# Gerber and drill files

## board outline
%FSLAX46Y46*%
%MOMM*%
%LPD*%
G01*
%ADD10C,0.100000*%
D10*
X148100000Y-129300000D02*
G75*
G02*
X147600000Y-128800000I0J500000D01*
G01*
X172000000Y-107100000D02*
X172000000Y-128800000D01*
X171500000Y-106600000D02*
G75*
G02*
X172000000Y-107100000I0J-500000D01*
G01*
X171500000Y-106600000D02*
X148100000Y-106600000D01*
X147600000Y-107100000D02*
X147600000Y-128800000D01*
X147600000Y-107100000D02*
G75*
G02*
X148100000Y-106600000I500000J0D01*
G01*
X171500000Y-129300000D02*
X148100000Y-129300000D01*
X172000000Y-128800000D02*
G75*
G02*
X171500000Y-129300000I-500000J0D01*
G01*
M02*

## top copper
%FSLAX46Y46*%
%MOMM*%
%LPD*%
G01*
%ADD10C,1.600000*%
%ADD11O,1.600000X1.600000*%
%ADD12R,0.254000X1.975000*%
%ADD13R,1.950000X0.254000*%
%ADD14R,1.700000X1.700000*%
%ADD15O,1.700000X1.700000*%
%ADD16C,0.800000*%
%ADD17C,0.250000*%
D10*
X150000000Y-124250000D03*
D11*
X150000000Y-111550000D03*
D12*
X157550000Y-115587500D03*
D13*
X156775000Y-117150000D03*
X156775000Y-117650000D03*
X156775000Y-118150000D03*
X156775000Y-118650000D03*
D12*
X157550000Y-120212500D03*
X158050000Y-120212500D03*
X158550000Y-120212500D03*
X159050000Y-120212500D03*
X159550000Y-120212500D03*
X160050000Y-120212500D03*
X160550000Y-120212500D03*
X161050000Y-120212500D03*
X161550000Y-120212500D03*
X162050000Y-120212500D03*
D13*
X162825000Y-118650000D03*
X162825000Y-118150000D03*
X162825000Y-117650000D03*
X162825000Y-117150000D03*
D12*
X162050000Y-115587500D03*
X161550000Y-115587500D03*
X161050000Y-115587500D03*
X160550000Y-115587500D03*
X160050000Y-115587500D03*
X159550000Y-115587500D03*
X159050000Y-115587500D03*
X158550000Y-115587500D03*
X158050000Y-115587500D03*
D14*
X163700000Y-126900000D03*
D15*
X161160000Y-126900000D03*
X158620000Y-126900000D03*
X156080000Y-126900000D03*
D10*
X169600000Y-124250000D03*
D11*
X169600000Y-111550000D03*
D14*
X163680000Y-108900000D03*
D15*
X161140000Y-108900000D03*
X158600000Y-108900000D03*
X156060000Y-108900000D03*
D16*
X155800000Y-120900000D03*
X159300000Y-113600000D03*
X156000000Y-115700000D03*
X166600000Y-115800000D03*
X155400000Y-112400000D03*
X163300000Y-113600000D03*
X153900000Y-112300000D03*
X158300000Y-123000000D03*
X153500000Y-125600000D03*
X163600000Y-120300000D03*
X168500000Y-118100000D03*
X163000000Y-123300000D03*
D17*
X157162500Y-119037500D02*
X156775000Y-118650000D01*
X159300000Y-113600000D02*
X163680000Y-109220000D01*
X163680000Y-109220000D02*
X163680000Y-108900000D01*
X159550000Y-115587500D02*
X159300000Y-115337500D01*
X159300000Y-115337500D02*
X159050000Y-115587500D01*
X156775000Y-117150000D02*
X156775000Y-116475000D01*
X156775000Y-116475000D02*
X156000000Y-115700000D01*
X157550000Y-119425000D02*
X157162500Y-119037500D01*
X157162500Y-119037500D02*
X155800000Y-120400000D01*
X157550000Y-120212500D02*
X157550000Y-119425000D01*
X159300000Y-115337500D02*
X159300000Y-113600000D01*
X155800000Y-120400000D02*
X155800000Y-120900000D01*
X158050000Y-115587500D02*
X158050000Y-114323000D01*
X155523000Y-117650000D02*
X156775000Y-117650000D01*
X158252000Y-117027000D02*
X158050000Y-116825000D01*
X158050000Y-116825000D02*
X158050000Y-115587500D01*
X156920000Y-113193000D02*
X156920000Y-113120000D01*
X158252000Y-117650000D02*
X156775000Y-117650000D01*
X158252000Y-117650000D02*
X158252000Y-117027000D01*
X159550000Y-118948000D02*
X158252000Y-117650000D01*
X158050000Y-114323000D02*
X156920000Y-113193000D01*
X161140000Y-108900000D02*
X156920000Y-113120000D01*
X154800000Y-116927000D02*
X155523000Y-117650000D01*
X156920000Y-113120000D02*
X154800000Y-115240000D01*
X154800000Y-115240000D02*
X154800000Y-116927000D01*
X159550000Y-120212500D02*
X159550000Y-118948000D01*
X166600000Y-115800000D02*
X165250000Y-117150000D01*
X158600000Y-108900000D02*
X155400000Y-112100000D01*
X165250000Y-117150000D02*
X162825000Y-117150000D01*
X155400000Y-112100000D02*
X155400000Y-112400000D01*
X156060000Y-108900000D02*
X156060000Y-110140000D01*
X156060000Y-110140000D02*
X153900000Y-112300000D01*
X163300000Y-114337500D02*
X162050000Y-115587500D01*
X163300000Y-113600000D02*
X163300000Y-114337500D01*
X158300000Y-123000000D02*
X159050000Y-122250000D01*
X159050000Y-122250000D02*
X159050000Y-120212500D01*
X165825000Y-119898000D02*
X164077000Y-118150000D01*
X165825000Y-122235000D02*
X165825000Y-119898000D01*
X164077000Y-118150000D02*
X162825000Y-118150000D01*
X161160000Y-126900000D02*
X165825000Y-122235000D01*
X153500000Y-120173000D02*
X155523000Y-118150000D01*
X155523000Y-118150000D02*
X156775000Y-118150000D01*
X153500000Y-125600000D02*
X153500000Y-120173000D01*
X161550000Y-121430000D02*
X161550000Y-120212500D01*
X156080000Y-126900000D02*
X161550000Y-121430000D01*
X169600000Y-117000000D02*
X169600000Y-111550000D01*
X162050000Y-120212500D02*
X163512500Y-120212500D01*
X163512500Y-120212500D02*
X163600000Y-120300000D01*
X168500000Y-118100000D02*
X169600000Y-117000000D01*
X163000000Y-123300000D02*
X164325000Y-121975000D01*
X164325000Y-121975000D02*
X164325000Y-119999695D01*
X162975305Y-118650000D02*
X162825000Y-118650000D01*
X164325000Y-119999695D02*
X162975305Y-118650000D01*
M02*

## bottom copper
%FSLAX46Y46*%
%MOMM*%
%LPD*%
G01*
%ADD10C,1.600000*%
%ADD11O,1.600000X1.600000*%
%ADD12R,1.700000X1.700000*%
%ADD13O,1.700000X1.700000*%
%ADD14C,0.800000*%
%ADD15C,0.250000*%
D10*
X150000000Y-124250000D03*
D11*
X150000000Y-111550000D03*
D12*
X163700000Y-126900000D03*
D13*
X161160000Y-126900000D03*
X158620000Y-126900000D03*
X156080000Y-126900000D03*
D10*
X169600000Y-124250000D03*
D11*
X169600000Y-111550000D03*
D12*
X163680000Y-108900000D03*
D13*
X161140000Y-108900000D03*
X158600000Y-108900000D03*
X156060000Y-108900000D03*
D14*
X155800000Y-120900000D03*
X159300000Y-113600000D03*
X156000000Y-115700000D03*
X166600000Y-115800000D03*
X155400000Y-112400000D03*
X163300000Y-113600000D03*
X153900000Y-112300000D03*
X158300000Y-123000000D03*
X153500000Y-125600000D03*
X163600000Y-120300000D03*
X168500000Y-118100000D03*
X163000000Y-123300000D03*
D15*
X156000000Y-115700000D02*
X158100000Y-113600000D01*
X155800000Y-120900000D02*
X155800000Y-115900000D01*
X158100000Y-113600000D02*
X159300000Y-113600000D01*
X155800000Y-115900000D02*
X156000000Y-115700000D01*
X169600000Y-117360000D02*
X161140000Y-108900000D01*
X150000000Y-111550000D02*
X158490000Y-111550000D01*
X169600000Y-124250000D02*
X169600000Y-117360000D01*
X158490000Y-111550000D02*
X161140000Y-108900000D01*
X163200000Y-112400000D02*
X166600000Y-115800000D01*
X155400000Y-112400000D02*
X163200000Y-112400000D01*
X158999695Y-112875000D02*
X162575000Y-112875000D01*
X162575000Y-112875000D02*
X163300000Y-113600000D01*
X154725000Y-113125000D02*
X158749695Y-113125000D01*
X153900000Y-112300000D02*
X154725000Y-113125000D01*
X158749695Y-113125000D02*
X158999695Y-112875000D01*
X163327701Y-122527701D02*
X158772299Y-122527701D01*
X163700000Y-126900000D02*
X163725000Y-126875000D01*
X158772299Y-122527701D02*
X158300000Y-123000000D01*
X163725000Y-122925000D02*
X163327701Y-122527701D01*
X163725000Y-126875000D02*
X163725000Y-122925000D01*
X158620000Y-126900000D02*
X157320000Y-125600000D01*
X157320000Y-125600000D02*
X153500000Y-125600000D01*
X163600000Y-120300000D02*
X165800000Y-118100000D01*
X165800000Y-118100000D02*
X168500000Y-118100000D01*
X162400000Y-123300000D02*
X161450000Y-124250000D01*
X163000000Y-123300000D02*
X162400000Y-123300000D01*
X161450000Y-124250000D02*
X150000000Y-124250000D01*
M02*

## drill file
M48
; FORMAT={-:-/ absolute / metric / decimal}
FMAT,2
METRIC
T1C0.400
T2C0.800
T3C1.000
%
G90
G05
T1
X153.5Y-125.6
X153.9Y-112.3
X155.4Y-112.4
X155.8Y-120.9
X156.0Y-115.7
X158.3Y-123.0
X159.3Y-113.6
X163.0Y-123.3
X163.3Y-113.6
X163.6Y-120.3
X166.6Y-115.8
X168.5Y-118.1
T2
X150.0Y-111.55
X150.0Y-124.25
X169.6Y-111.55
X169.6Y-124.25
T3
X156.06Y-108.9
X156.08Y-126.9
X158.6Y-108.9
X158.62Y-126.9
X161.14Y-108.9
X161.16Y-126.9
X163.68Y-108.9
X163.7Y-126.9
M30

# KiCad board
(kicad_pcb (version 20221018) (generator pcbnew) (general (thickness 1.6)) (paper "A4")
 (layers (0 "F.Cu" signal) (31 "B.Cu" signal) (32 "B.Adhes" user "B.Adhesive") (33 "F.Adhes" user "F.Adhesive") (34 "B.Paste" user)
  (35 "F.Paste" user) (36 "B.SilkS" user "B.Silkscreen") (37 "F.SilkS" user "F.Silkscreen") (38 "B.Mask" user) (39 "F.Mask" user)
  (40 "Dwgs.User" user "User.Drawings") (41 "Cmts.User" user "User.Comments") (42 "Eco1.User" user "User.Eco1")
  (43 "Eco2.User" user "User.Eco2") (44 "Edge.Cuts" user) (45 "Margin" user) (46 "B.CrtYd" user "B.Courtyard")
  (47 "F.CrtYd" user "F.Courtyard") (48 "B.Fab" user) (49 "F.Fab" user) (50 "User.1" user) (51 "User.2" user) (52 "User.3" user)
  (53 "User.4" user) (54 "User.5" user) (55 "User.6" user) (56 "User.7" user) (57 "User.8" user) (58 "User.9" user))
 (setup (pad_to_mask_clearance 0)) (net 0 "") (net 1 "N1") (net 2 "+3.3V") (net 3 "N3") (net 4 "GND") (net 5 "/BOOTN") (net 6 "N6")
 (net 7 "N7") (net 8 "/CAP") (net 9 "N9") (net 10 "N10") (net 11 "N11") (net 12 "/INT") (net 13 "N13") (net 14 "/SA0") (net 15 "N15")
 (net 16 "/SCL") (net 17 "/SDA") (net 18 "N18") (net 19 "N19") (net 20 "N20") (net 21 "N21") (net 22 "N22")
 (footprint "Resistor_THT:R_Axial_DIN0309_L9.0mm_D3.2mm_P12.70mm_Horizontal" (layer "F.Cu") (at 150 124.25 90)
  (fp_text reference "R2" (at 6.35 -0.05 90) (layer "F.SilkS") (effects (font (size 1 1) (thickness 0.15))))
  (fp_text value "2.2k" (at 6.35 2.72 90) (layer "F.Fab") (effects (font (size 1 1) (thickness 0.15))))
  (pad "1" thru_hole circle (at 0 0 90) (size 1.6 1.6) (drill 0.8) (layers "*.Cu" "*.Mask") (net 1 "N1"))
  (pad "2" thru_hole oval (at 12.7 0 90) (size 1.6 1.6) (drill 0.8) (layers "*.Cu" "*.Mask") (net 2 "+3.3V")))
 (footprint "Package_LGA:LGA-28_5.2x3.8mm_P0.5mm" (layer "F.Cu") (at 159.8 117.9)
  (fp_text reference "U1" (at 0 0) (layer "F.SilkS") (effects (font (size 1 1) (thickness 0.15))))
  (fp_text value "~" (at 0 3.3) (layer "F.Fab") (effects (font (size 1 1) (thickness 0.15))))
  (pad "1" smd rect (at -2.25 -2.3125) (size 0.254 1.975) (layers "F.Cu" "F.Paste" "F.Mask") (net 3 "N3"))
  (pad "2" smd rect (at -3.025 -0.75 90) (size 0.254 1.95) (layers "F.Cu" "F.Paste" "F.Mask") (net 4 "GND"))
  (pad "3" smd rect (at -3.025 -0.25 90) (size 0.254 1.95) (layers "F.Cu" "F.Paste" "F.Mask") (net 2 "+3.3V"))
  (pad "4" smd rect (at -3.025 0.25 90) (size 0.254 1.95) (layers "F.Cu" "F.Paste" "F.Mask") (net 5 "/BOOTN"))
  (pad "5" smd rect (at -3.025 0.75 90) (size 0.254 1.95) (layers "F.Cu" "F.Paste" "F.Mask") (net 4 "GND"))
  (pad "6" smd rect (at -2.25 2.3125) (size 0.254 1.975) (layers "F.Cu" "F.Paste" "F.Mask") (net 4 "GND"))
  (pad "7" smd rect (at -1.75 2.3125) (size 0.254 1.975) (layers "F.Cu" "F.Paste" "F.Mask") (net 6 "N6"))
  (pad "8" smd rect (at -1.25 2.3125) (size 0.254 1.975) (layers "F.Cu" "F.Paste" "F.Mask") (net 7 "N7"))
  (pad "9" smd rect (at -0.75 2.3125) (size 0.254 1.975) (layers "F.Cu" "F.Paste" "F.Mask") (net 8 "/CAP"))
  (pad "10" smd rect (at -0.25 2.3125) (size 0.254 1.975) (layers "F.Cu" "F.Paste" "F.Mask") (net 2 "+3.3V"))
  (pad "11" smd rect (at 0.25 2.3125) (size 0.254 1.975) (layers "F.Cu" "F.Paste" "F.Mask") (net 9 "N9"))
  (pad "12" smd rect (at 0.75 2.3125) (size 0.254 1.975) (layers "F.Cu" "F.Paste" "F.Mask") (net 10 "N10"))
  (pad "13" smd rect (at 1.25 2.3125) (size 0.254 1.975) (layers "F.Cu" "F.Paste" "F.Mask") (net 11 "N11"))
  (pad "14" smd rect (at 1.75 2.3125) (size 0.254 1.975) (layers "F.Cu" "F.Paste" "F.Mask") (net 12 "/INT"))
  (pad "15" smd rect (at 2.25 2.3125) (size 0.254 1.975) (layers "F.Cu" "F.Paste" "F.Mask") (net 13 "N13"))
  (pad "16" smd rect (at 3.025 0.75 90) (size 0.254 1.95) (layers "F.Cu" "F.Paste" "F.Mask") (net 1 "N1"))
  (pad "17" smd rect (at 3.025 0.25 90) (size 0.254 1.95) (layers "F.Cu" "F.Paste" "F.Mask") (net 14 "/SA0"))
  (pad "18" smd rect (at 3.025 -0.25 90) (size 0.254 1.95) (layers "F.Cu" "F.Paste" "F.Mask") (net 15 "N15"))
  (pad "19" smd rect (at 3.025 -0.75 90) (size 0.254 1.95) (layers "F.Cu" "F.Paste" "F.Mask") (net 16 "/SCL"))
  (pad "20" smd rect (at 2.25 -2.3125) (size 0.254 1.975) (layers "F.Cu" "F.Paste" "F.Mask") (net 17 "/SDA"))
  (pad "21" smd rect (at 1.75 -2.3125) (size 0.254 1.975) (layers "F.Cu" "F.Paste" "F.Mask") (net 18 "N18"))
  (pad "22" smd rect (at 1.25 -2.3125) (size 0.254 1.975) (layers "F.Cu" "F.Paste" "F.Mask") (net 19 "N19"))
  (pad "23" smd rect (at 0.75 -2.3125) (size 0.254 1.975) (layers "F.Cu" "F.Paste" "F.Mask") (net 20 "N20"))
  (pad "24" smd rect (at 0.25 -2.3125) (size 0.254 1.975) (layers "F.Cu" "F.Paste" "F.Mask") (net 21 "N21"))
  (pad "25" smd rect (at -0.25 -2.3125) (size 0.254 1.975) (layers "F.Cu" "F.Paste" "F.Mask") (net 4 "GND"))
  (pad "26" smd rect (at -0.75 -2.3125) (size 0.254 1.975) (layers "F.Cu" "F.Paste" "F.Mask") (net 4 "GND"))
  (pad "27" smd rect (at -1.25 -2.3125) (size 0.254 1.975) (layers "F.Cu" "F.Paste" "F.Mask") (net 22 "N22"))
  (pad "28" smd rect (at -1.75 -2.3125) (size 0.254 1.975) (layers "F.Cu" "F.Paste" "F.Mask") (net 2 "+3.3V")))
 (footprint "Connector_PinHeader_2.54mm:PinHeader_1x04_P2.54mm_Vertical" (layer "F.Cu") (at 163.7 126.9 -90)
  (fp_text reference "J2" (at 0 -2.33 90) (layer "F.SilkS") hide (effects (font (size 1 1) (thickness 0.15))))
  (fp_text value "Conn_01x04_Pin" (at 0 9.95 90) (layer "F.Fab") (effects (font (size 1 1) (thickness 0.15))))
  (pad "1" thru_hole rect (at 0 0 270) (size 1.7 1.7) (drill 1) (layers "*.Cu" "*.Mask") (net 8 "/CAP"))
  (pad "2" thru_hole oval (at 0 2.54 270) (size 1.7 1.7) (drill 1) (layers "*.Cu" "*.Mask") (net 14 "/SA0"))
  (pad "3" thru_hole oval (at 0 5.08 270) (size 1.7 1.7) (drill 1) (layers "*.Cu" "*.Mask") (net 5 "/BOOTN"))
  (pad "4" thru_hole oval (at 0 7.62 270) (size 1.7 1.7) (drill 1) (layers "*.Cu" "*.Mask") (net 12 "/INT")))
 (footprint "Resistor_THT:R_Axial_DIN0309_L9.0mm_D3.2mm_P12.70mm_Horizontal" (layer "F.Cu") (at 169.6 124.25 90)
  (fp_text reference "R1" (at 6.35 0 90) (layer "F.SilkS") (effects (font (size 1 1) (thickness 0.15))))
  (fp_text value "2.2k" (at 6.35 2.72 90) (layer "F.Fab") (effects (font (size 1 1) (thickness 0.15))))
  (pad "1" thru_hole circle (at 0 0 90) (size 1.6 1.6) (drill 0.8) (layers "*.Cu" "*.Mask") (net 2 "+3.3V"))
  (pad "2" thru_hole oval (at 12.7 0 90) (size 1.6 1.6) (drill 0.8) (layers "*.Cu" "*.Mask") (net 13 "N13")))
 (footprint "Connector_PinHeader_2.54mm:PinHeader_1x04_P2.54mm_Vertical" (layer "F.Cu") (at 163.68 108.9 -90)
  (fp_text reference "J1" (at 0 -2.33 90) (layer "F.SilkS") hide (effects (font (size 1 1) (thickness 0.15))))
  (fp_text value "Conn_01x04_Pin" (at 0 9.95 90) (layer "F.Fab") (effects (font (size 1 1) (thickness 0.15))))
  (pad "1" thru_hole rect (at 0 0 270) (size 1.7 1.7) (drill 1) (layers "*.Cu" "*.Mask") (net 4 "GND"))
  (pad "2" thru_hole oval (at 0 2.54 270) (size 1.7 1.7) (drill 1) (layers "*.Cu" "*.Mask") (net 2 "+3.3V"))
  (pad "3" thru_hole oval (at 0 5.08 270) (size 1.7 1.7) (drill 1) (layers "*.Cu" "*.Mask") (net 16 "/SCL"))
  (pad "4" thru_hole oval (at 0 7.62 270) (size 1.7 1.7) (drill 1) (layers "*.Cu" "*.Mask") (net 17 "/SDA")))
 (gr_arc (start 148.1 129.3) (mid 147.746447 129.153553) (end 147.6 128.8) (stroke (width 0.1) (type default)) (layer "Edge.Cuts"))
 (gr_line (start 172 107.1) (end 172 128.8) (stroke (width 0.1) (type default)) (layer "Edge.Cuts"))
 (gr_arc (start 171.5 106.6) (mid 171.853553 106.746447) (end 172 107.1) (stroke (width 0.1) (type default)) (layer "Edge.Cuts"))
 (gr_line (start 171.5 106.6) (end 148.1 106.6) (stroke (width 0.1) (type default)) (layer "Edge.Cuts"))
 (gr_line (start 147.6 107.1) (end 147.6 128.8) (stroke (width 0.1) (type default)) (layer "Edge.Cuts"))
 (gr_arc (start 147.6 107.1) (mid 147.746447 106.746447) (end 148.1 106.6) (stroke (width 0.1) (type default)) (layer "Edge.Cuts"))
 (gr_line (start 171.5 129.3) (end 148.1 129.3) (stroke (width 0.1) (type default)) (layer "Edge.Cuts"))
 (gr_arc (start 172 128.8) (mid 171.853553 129.153553) (end 171.5 129.3) (stroke (width 0.1) (type default)) (layer "Edge.Cuts"))
 (segment (start 157.1625 119.0375) (end 156.775 118.65) (width 0.25) (layer "F.Cu") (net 4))
 (segment (start 159.3 113.6) (end 163.68 109.22) (width 0.25) (layer "F.Cu") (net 4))
 (segment (start 163.68 109.22) (end 163.68 108.9) (width 0.25) (layer "F.Cu") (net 4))
 (segment (start 159.55 115.5875) (end 159.3 115.3375) (width 0.25) (layer "F.Cu") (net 4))
 (segment (start 159.3 115.3375) (end 159.05 115.5875) (width 0.25) (layer "F.Cu") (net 4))
 (segment (start 156.775 117.15) (end 156.775 116.475) (width 0.25) (layer "F.Cu") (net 4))
 (segment (start 156.775 116.475) (end 156 115.7) (width 0.25) (layer "F.Cu") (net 4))
 (segment (start 157.55 119.425) (end 157.1625 119.0375) (width 0.25) (layer "F.Cu") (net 4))
 (segment (start 157.1625 119.0375) (end 155.8 120.4) (width 0.25) (layer "F.Cu") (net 4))
 (segment (start 157.55 120.2125) (end 157.55 119.425) (width 0.25) (layer "F.Cu") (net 4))
 (segment (start 159.3 115.3375) (end 159.3 113.6) (width 0.25) (layer "F.Cu") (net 4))
 (segment (start 155.8 120.4) (end 155.8 120.9) (width 0.25) (layer "F.Cu") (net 4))
 (via (at 155.8 120.9) (size 0.8) (drill 0.4) (layers "F.Cu" "B.Cu") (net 4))
 (via (at 159.3 113.6) (size 0.8) (drill 0.4) (layers "F.Cu" "B.Cu") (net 4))
 (via (at 156 115.7) (size 0.8) (drill 0.4) (layers "F.Cu" "B.Cu") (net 4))
 (segment (start 156 115.7) (end 158.1 113.6) (width 0.25) (layer "B.Cu") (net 4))
 (segment (start 155.8 120.9) (end 155.8 115.9) (width 0.25) (layer "B.Cu") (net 4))
 (segment (start 158.1 113.6) (end 159.3 113.6) (width 0.25) (layer "B.Cu") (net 4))
 (segment (start 155.8 115.9) (end 156 115.7) (width 0.25) (layer "B.Cu") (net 4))
 (segment (start 158.05 115.5875) (end 158.05 114.323) (width 0.25) (layer "F.Cu") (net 2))
 (segment (start 155.523 117.65) (end 156.775 117.65) (width 0.25) (layer "F.Cu") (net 2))
 (segment (start 158.252 117.027) (end 158.05 116.825) (width 0.25) (layer "F.Cu") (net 2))
 (segment (start 158.05 116.825) (end 158.05 115.5875) (width 0.25) (layer "F.Cu") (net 2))
 (segment (start 156.92 113.193) (end 156.92 113.12) (width 0.25) (layer "F.Cu") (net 2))
 (segment (start 158.252 117.65) (end 156.775 117.65) (width 0.25) (layer "F.Cu") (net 2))
 (segment (start 158.252 117.65) (end 158.252 117.027) (width 0.25) (layer "F.Cu") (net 2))
 (segment (start 159.55 118.948) (end 158.252 117.65) (width 0.25) (layer "F.Cu") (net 2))
 (segment (start 158.05 114.323) (end 156.92 113.193) (width 0.25) (layer "F.Cu") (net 2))
 (segment (start 161.14 108.9) (end 156.92 113.12) (width 0.25) (layer "F.Cu") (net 2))
 (segment (start 154.8 116.927) (end 155.523 117.65) (width 0.25) (layer "F.Cu") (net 2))
 (segment (start 156.92 113.12) (end 154.8 115.24) (width 0.25) (layer "F.Cu") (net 2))
 (segment (start 154.8 115.24) (end 154.8 116.927) (width 0.25) (layer "F.Cu") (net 2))
 (segment (start 159.55 120.2125) (end 159.55 118.948) (width 0.25) (layer "F.Cu") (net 2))
 (segment (start 169.6 117.36) (end 161.14 108.9) (width 0.25) (layer "B.Cu") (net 2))
 (segment (start 150 111.55) (end 158.49 111.55) (width 0.25) (layer "B.Cu") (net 2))
 (segment (start 169.6 124.25) (end 169.6 117.36) (width 0.25) (layer "B.Cu") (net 2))
 (segment (start 158.49 111.55) (end 161.14 108.9) (width 0.25) (layer "B.Cu") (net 2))
 (segment (start 166.6 115.8) (end 165.25 117.15) (width 0.25) (layer "F.Cu") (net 16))
 (segment (start 158.6 108.9) (end 155.4 112.1) (width 0.25) (layer "F.Cu") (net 16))
 (segment (start 165.25 117.15) (end 162.825 117.15) (width 0.25) (layer "F.Cu") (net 16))
 (segment (start 155.4 112.1) (end 155.4 112.4) (width 0.25) (layer "F.Cu") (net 16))
 (via (at 166.6 115.8) (size 0.8) (drill 0.4) (layers "F.Cu" "B.Cu") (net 16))
 (via (at 155.4 112.4) (size 0.8) (drill 0.4) (layers "F.Cu" "B.Cu") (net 16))
 (segment (start 163.2 112.4) (end 166.6 115.8) (width 0.25) (layer "B.Cu") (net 16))
 (segment (start 155.4 112.4) (end 163.2 112.4) (width 0.25) (layer "B.Cu") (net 16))
 (segment (start 156.06 108.9) (end 156.06 110.14) (width 0.25) (layer "F.Cu") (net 17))
 (segment (start 156.06 110.14) (end 153.9 112.3) (width 0.25) (layer "F.Cu") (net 17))
 (segment (start 163.3 114.3375) (end 162.05 115.5875) (width 0.25) (layer "F.Cu") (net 17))
 (segment (start 163.3 113.6) (end 163.3 114.3375) (width 0.25) (layer "F.Cu") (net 17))
 (via (at 163.3 113.6) (size 0.8) (drill 0.4) (layers "F.Cu" "B.Cu") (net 17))
 (via (at 153.9 112.3) (size 0.8) (drill 0.4) (layers "F.Cu" "B.Cu") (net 17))
 (segment (start 158.999695 112.875) (end 162.575 112.875) (width 0.25) (layer "B.Cu") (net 17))
 (segment (start 162.575 112.875) (end 163.3 113.6) (width 0.25) (layer "B.Cu") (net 17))
 (segment (start 154.725 113.125) (end 158.749695 113.125) (width 0.25) (layer "B.Cu") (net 17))
 (segment (start 153.9 112.3) (end 154.725 113.125) (width 0.25) (layer "B.Cu") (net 17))
 (segment (start 158.749695 113.125) (end 158.999695 112.875) (width 0.25) (layer "B.Cu") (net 17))
 (segment (start 158.3 123) (end 159.05 122.25) (width 0.25) (layer "F.Cu") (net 8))
 (segment (start 159.05 122.25) (end 159.05 120.2125) (width 0.25) (layer "F.Cu") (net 8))
 (via (at 158.3 123) (size 0.8) (drill 0.4) (layers "F.Cu" "B.Cu") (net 8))
 (segment (start 163.327701 122.527701) (end 158.772299 122.527701) (width 0.25) (layer "B.Cu") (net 8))
 (segment (start 163.7 126.9) (end 163.725 126.875) (width 0.25) (layer "B.Cu") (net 8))
 (segment (start 158.772299 122.527701) (end 158.3 123) (width 0.25) (layer "B.Cu") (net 8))
 (segment (start 163.725 122.925) (end 163.327701 122.527701) (width 0.25) (layer "B.Cu") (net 8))
 (segment (start 163.725 126.875) (end 163.725 122.925) (width 0.25) (layer "B.Cu") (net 8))
 (segment (start 165.825 119.898) (end 164.077 118.15) (width 0.25) (layer "F.Cu") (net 14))
 (segment (start 165.825 122.235) (end 165.825 119.898) (width 0.25) (layer "F.Cu") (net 14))
 (segment (start 164.077 118.15) (end 162.825 118.15) (width 0.25) (layer "F.Cu") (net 14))
 (segment (start 161.16 126.9) (end 165.825 122.235) (width 0.25) (layer "F.Cu") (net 14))
 (segment (start 153.5 120.173) (end 155.523 118.15) (width 0.25) (layer "F.Cu") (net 5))
 (segment (start 155.523 118.15) (end 156.775 118.15) (width 0.25) (layer "F.Cu") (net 5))
 (segment (start 153.5 125.6) (end 153.5 120.173) (width 0.25) (layer "F.Cu") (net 5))
 (via (at 153.5 125.6) (size 0.8) (drill 0.4) (layers "F.Cu" "B.Cu") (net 5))
 (segment (start 158.62 126.9) (end 157.32 125.6) (width 0.25) (layer "B.Cu") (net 5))
 (segment (start 157.32 125.6) (end 153.5 125.6) (width 0.25) (layer "B.Cu") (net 5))
 (segment (start 161.55 121.43) (end 161.55 120.2125) (width 0.25) (layer "F.Cu") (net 12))
 (segment (start 156.08 126.9) (end 161.55 121.43) (width 0.25) (layer "F.Cu") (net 12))
 (segment (start 169.6 117) (end 169.6 111.55) (width 0.25) (layer "F.Cu") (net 13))
 (segment (start 162.05 120.2125) (end 163.5125 120.2125) (width 0.25) (layer "F.Cu") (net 13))
 (segment (start 163.5125 120.2125) (end 163.6 120.3) (width 0.25) (layer "F.Cu") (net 13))
 (segment (start 168.5 118.1) (end 169.6 117) (width 0.25) (layer "F.Cu") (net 13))
 (via (at 163.6 120.3) (size 0.8) (drill 0.4) (layers "F.Cu" "B.Cu") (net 13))
 (via (at 168.5 118.1) (size 0.8) (drill 0.4) (layers "F.Cu" "B.Cu") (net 13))
 (segment (start 163.6 120.3) (end 165.8 118.1) (width 0.25) (layer "B.Cu") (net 13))
 (segment (start 165.8 118.1) (end 168.5 118.1) (width 0.25) (layer "B.Cu") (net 13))
 (segment (start 163 123.3) (end 164.325 121.975) (width 0.25) (layer "F.Cu") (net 1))
 (segment (start 164.325 121.975) (end 164.325 119.999695) (width 0.25) (layer "F.Cu") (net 1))
 (segment (start 162.975305 118.65) (end 162.825 118.65) (width 0.25) (layer "F.Cu") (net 1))
 (segment (start 164.325 119.999695) (end 162.975305 118.65) (width 0.25) (layer "F.Cu") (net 1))
 (via (at 163 123.3) (size 0.8) (drill 0.4) (layers "F.Cu" "B.Cu") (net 1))
 (segment (start 162.4 123.3) (end 161.45 124.25) (width 0.25) (layer "B.Cu") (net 1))
 (segment (start 163 123.3) (end 162.4 123.3) (width 0.25) (layer "B.Cu") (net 1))
 (segment (start 161.45 124.25) (end 150 124.25) (width 0.25) (layer "B.Cu") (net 1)))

